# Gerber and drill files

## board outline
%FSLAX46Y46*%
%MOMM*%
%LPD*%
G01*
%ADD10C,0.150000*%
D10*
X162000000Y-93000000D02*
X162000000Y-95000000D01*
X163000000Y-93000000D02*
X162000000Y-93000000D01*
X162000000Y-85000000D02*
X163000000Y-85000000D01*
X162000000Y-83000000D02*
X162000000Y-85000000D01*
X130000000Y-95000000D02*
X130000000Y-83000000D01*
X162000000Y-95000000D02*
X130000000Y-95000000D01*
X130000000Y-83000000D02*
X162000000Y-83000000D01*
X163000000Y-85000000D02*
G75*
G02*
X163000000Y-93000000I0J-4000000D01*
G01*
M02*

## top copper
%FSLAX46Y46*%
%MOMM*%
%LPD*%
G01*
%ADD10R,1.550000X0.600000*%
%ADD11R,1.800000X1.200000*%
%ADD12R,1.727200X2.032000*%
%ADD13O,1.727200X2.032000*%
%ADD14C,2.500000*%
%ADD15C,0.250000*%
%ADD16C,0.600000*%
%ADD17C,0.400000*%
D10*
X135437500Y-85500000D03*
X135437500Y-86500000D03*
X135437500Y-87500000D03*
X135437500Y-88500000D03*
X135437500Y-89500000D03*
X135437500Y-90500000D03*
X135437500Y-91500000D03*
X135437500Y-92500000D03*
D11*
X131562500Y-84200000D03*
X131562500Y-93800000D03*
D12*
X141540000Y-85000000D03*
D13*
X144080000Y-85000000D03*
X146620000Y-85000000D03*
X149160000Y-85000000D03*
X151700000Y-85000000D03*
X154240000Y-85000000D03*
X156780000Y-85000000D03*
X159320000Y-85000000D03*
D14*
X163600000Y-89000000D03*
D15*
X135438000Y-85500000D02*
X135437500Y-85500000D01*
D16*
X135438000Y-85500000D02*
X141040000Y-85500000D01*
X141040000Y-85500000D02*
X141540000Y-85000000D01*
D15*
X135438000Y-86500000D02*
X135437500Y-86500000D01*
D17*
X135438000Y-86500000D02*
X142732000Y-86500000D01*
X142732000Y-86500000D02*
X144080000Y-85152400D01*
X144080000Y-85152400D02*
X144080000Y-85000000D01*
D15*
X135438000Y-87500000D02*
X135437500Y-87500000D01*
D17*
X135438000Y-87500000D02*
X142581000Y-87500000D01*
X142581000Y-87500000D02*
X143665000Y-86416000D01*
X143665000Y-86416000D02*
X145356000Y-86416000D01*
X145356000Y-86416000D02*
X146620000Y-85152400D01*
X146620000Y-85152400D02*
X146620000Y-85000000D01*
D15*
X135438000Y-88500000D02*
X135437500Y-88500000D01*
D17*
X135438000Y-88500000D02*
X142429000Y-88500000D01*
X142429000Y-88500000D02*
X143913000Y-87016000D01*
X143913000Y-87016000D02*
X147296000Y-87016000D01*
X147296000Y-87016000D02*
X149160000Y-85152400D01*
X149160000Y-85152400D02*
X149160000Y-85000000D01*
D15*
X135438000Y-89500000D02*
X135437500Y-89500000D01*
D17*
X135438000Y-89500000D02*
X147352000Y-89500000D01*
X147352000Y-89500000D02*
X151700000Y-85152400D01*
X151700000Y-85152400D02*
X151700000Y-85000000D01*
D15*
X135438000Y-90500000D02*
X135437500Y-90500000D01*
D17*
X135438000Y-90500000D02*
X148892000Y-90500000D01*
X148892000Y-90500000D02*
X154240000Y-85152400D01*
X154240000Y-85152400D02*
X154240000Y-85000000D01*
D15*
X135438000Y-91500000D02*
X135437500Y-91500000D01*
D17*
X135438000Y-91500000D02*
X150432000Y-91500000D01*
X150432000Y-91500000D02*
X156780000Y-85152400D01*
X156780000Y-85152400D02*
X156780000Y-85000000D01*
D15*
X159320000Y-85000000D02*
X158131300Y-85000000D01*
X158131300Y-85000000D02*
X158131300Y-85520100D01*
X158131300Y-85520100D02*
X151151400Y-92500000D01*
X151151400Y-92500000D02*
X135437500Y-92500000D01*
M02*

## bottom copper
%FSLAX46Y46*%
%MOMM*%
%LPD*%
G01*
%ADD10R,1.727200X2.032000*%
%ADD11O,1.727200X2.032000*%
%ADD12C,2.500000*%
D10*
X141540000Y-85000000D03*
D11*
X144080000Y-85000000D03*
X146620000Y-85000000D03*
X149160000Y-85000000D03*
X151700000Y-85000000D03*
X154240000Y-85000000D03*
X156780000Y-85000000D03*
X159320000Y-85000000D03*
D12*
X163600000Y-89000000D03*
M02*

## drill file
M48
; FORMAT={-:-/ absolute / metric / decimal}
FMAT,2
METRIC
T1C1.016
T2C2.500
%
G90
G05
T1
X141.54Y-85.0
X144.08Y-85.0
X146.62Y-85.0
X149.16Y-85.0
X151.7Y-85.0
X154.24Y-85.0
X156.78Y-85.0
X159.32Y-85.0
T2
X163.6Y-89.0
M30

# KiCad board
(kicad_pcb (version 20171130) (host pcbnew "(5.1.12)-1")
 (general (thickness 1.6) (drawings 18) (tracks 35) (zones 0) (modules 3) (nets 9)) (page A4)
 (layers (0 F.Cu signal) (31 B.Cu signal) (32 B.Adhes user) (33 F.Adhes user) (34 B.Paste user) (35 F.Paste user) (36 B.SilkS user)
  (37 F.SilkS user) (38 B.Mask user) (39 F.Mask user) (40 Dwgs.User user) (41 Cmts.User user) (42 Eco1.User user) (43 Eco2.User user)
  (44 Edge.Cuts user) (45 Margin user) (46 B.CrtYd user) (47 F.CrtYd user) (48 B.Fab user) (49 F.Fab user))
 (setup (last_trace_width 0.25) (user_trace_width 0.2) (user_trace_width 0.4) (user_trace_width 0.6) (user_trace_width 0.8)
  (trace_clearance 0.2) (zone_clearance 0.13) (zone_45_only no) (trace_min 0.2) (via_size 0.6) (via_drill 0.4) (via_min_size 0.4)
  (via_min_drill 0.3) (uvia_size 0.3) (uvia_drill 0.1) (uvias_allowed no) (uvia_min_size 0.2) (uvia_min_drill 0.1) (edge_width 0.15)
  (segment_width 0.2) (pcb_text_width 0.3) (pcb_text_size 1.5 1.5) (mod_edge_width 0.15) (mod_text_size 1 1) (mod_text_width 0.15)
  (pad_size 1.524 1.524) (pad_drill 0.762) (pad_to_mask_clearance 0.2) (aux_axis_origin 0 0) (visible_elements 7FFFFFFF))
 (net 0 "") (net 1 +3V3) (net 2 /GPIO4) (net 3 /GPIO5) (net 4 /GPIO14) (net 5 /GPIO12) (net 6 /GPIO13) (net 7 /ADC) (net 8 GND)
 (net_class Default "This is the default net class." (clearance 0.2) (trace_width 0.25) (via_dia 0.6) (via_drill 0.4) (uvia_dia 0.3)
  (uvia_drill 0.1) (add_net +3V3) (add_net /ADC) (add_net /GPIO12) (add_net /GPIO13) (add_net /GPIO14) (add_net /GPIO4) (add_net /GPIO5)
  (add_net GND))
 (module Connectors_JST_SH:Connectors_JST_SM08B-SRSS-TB (layer F.Cu) (at 133.5 89 270)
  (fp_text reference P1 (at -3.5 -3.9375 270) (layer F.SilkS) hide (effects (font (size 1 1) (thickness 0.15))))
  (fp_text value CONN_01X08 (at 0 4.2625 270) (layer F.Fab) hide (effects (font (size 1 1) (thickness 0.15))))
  (pad 1 smd rect (at -3.5 -1.9375 270) (size 0.6 1.55) (layers F.Cu F.Paste F.Mask) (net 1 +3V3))
  (pad 2 smd rect (at -2.5 -1.9375 270) (size 0.6 1.55) (layers F.Cu F.Paste F.Mask) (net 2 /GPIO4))
  (pad 3 smd rect (at -1.5 -1.9375 270) (size 0.6 1.55) (layers F.Cu F.Paste F.Mask) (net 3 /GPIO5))
  (pad 4 smd rect (at -0.5 -1.9375 270) (size 0.6 1.55) (layers F.Cu F.Paste F.Mask) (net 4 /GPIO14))
  (pad 5 smd rect (at 0.5 -1.9375 270) (size 0.6 1.55) (layers F.Cu F.Paste F.Mask) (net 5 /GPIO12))
  (pad 6 smd rect (at 1.5 -1.9375 270) (size 0.6 1.55) (layers F.Cu F.Paste F.Mask) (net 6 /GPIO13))
  (pad 7 smd rect (at 2.5 -1.9375 270) (size 0.6 1.55) (layers F.Cu F.Paste F.Mask) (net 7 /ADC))
  (pad 8 smd rect (at 3.5 -1.9375 270) (size 0.6 1.55) (layers F.Cu F.Paste F.Mask) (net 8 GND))
  (pad "" smd rect (at -4.8 1.9375 270) (size 1.2 1.8) (layers F.Cu F.Paste F.Mask))
  (pad "" smd rect (at 4.8 1.9375 270) (size 1.2 1.8) (layers F.Cu F.Paste F.Mask)))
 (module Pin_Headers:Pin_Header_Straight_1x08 (layer F.Cu) (at 141.54 85 90)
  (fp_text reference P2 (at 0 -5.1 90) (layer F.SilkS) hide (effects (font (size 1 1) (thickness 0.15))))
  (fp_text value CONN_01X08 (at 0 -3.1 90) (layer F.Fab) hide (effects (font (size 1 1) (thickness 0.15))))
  (pad 1 thru_hole rect (at 0 0 90) (size 2.032 1.7272) (drill 1.016) (layers *.Cu *.Mask F.SilkS) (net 1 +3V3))
  (pad 2 thru_hole oval (at 0 2.54 90) (size 2.032 1.7272) (drill 1.016) (layers *.Cu *.Mask F.SilkS) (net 2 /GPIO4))
  (pad 3 thru_hole oval (at 0 5.08 90) (size 2.032 1.7272) (drill 1.016) (layers *.Cu *.Mask F.SilkS) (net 3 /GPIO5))
  (pad 4 thru_hole oval (at 0 7.62 90) (size 2.032 1.7272) (drill 1.016) (layers *.Cu *.Mask F.SilkS) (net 4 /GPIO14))
  (pad 5 thru_hole oval (at 0 10.16 90) (size 2.032 1.7272) (drill 1.016) (layers *.Cu *.Mask F.SilkS) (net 5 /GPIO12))
  (pad 6 thru_hole oval (at 0 12.7 90) (size 2.032 1.7272) (drill 1.016) (layers *.Cu *.Mask F.SilkS) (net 6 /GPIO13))
  (pad 7 thru_hole oval (at 0 15.24 90) (size 2.032 1.7272) (drill 1.016) (layers *.Cu *.Mask F.SilkS) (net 7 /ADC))
  (pad 8 thru_hole oval (at 0 17.78 90) (size 2.032 1.7272) (drill 1.016) (layers *.Cu *.Mask F.SilkS) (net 8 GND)))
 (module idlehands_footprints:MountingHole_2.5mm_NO (layer F.Cu) (at 163.625 89)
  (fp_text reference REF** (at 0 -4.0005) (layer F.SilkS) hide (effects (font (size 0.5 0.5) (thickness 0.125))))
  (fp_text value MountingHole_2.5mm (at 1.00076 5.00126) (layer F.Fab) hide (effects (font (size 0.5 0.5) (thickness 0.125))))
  (pad 1 thru_hole circle (at -0.025 0) (size 2.5 2.5) (drill 2.5) (layers *.Cu)))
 (gr_line (start 162 93) (end 162 95) (layer Edge.Cuts) (width 0.15))
 (gr_line (start 163 93) (end 162 93) (layer Edge.Cuts) (width 0.15))
 (gr_line (start 162 85) (end 163 85) (layer Edge.Cuts) (width 0.15))
 (gr_line (start 162 83) (end 162 85) (layer Edge.Cuts) (width 0.15))
 (gr_line (start 130 95) (end 130 83) (layer Edge.Cuts) (width 0.15))
 (gr_line (start 162 95) (end 130 95) (layer Edge.Cuts) (width 0.15))
 (gr_line (start 130 83) (end 162 83) (layer Edge.Cuts) (width 0.15))
 (gr_arc (start 163 89) (end 163 85) (angle 180) (layer Edge.Cuts) (width 0.15))
 (segment (start 135.438 85.5) (end 135.4375 85.5) (width 0.25) (layer F.Cu) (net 1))
 (segment (start 135.438 85.5) (end 141.04 85.5) (width 0.6) (layer F.Cu) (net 1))
 (segment (start 141.04 85.5) (end 141.54 85) (width 0.6) (layer F.Cu) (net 1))
 (segment (start 135.438 86.5) (end 135.4375 86.5) (width 0.25) (layer F.Cu) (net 2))
 (segment (start 135.438 86.5) (end 142.732 86.5) (width 0.4) (layer F.Cu) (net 2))
 (segment (start 142.732 86.5) (end 144.08 85.1524) (width 0.4) (layer F.Cu) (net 2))
 (segment (start 144.08 85.1524) (end 144.08 85) (width 0.4) (layer F.Cu) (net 2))
 (segment (start 135.438 87.5) (end 135.4375 87.5) (width 0.25) (layer F.Cu) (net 3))
 (segment (start 135.438 87.5) (end 142.581 87.5) (width 0.4) (layer F.Cu) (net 3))
 (segment (start 142.581 87.5) (end 143.665 86.416) (width 0.4) (layer F.Cu) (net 3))
 (segment (start 143.665 86.416) (end 145.356 86.416) (width 0.4) (layer F.Cu) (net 3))
 (segment (start 145.356 86.416) (end 146.62 85.1524) (width 0.4) (layer F.Cu) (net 3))
 (segment (start 146.62 85.1524) (end 146.62 85) (width 0.4) (layer F.Cu) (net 3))
 (segment (start 135.438 88.5) (end 135.4375 88.5) (width 0.25) (layer F.Cu) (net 4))
 (segment (start 135.438 88.5) (end 142.429 88.5) (width 0.4) (layer F.Cu) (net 4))
 (segment (start 142.429 88.5) (end 143.913 87.016) (width 0.4) (layer F.Cu) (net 4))
 (segment (start 143.913 87.016) (end 147.296 87.016) (width 0.4) (layer F.Cu) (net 4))
 (segment (start 147.296 87.016) (end 149.16 85.1524) (width 0.4) (layer F.Cu) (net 4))
 (segment (start 149.16 85.1524) (end 149.16 85) (width 0.4) (layer F.Cu) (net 4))
 (segment (start 135.438 89.5) (end 135.4375 89.5) (width 0.25) (layer F.Cu) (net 5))
 (segment (start 135.438 89.5) (end 147.352 89.5) (width 0.4) (layer F.Cu) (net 5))
 (segment (start 147.352 89.5) (end 151.7 85.1524) (width 0.4) (layer F.Cu) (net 5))
 (segment (start 151.7 85.1524) (end 151.7 85) (width 0.4) (layer F.Cu) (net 5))
 (segment (start 135.438 90.5) (end 135.4375 90.5) (width 0.25) (layer F.Cu) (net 6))
 (segment (start 135.438 90.5) (end 148.892 90.5) (width 0.4) (layer F.Cu) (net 6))
 (segment (start 148.892 90.5) (end 154.24 85.1524) (width 0.4) (layer F.Cu) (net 6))
 (segment (start 154.24 85.1524) (end 154.24 85) (width 0.4) (layer F.Cu) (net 6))
 (segment (start 135.438 91.5) (end 135.4375 91.5) (width 0.25) (layer F.Cu) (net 7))
 (segment (start 135.438 91.5) (end 150.432 91.5) (width 0.4) (layer F.Cu) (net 7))
 (segment (start 150.432 91.5) (end 156.78 85.1524) (width 0.4) (layer F.Cu) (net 7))
 (segment (start 156.78 85.1524) (end 156.78 85) (width 0.4) (layer F.Cu) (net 7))
 (segment (start 159.32 85) (end 158.1313 85) (width 0.25) (layer F.Cu) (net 8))
 (segment (start 158.1313 85) (end 158.1313 85.5201) (width 0.25) (layer F.Cu) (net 8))
 (segment (start 158.1313 85.5201) (end 151.1514 92.5) (width 0.25) (layer F.Cu) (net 8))
 (segment (start 151.1514 92.5) (end 135.4375 92.5) (width 0.25) (layer F.Cu) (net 8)))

